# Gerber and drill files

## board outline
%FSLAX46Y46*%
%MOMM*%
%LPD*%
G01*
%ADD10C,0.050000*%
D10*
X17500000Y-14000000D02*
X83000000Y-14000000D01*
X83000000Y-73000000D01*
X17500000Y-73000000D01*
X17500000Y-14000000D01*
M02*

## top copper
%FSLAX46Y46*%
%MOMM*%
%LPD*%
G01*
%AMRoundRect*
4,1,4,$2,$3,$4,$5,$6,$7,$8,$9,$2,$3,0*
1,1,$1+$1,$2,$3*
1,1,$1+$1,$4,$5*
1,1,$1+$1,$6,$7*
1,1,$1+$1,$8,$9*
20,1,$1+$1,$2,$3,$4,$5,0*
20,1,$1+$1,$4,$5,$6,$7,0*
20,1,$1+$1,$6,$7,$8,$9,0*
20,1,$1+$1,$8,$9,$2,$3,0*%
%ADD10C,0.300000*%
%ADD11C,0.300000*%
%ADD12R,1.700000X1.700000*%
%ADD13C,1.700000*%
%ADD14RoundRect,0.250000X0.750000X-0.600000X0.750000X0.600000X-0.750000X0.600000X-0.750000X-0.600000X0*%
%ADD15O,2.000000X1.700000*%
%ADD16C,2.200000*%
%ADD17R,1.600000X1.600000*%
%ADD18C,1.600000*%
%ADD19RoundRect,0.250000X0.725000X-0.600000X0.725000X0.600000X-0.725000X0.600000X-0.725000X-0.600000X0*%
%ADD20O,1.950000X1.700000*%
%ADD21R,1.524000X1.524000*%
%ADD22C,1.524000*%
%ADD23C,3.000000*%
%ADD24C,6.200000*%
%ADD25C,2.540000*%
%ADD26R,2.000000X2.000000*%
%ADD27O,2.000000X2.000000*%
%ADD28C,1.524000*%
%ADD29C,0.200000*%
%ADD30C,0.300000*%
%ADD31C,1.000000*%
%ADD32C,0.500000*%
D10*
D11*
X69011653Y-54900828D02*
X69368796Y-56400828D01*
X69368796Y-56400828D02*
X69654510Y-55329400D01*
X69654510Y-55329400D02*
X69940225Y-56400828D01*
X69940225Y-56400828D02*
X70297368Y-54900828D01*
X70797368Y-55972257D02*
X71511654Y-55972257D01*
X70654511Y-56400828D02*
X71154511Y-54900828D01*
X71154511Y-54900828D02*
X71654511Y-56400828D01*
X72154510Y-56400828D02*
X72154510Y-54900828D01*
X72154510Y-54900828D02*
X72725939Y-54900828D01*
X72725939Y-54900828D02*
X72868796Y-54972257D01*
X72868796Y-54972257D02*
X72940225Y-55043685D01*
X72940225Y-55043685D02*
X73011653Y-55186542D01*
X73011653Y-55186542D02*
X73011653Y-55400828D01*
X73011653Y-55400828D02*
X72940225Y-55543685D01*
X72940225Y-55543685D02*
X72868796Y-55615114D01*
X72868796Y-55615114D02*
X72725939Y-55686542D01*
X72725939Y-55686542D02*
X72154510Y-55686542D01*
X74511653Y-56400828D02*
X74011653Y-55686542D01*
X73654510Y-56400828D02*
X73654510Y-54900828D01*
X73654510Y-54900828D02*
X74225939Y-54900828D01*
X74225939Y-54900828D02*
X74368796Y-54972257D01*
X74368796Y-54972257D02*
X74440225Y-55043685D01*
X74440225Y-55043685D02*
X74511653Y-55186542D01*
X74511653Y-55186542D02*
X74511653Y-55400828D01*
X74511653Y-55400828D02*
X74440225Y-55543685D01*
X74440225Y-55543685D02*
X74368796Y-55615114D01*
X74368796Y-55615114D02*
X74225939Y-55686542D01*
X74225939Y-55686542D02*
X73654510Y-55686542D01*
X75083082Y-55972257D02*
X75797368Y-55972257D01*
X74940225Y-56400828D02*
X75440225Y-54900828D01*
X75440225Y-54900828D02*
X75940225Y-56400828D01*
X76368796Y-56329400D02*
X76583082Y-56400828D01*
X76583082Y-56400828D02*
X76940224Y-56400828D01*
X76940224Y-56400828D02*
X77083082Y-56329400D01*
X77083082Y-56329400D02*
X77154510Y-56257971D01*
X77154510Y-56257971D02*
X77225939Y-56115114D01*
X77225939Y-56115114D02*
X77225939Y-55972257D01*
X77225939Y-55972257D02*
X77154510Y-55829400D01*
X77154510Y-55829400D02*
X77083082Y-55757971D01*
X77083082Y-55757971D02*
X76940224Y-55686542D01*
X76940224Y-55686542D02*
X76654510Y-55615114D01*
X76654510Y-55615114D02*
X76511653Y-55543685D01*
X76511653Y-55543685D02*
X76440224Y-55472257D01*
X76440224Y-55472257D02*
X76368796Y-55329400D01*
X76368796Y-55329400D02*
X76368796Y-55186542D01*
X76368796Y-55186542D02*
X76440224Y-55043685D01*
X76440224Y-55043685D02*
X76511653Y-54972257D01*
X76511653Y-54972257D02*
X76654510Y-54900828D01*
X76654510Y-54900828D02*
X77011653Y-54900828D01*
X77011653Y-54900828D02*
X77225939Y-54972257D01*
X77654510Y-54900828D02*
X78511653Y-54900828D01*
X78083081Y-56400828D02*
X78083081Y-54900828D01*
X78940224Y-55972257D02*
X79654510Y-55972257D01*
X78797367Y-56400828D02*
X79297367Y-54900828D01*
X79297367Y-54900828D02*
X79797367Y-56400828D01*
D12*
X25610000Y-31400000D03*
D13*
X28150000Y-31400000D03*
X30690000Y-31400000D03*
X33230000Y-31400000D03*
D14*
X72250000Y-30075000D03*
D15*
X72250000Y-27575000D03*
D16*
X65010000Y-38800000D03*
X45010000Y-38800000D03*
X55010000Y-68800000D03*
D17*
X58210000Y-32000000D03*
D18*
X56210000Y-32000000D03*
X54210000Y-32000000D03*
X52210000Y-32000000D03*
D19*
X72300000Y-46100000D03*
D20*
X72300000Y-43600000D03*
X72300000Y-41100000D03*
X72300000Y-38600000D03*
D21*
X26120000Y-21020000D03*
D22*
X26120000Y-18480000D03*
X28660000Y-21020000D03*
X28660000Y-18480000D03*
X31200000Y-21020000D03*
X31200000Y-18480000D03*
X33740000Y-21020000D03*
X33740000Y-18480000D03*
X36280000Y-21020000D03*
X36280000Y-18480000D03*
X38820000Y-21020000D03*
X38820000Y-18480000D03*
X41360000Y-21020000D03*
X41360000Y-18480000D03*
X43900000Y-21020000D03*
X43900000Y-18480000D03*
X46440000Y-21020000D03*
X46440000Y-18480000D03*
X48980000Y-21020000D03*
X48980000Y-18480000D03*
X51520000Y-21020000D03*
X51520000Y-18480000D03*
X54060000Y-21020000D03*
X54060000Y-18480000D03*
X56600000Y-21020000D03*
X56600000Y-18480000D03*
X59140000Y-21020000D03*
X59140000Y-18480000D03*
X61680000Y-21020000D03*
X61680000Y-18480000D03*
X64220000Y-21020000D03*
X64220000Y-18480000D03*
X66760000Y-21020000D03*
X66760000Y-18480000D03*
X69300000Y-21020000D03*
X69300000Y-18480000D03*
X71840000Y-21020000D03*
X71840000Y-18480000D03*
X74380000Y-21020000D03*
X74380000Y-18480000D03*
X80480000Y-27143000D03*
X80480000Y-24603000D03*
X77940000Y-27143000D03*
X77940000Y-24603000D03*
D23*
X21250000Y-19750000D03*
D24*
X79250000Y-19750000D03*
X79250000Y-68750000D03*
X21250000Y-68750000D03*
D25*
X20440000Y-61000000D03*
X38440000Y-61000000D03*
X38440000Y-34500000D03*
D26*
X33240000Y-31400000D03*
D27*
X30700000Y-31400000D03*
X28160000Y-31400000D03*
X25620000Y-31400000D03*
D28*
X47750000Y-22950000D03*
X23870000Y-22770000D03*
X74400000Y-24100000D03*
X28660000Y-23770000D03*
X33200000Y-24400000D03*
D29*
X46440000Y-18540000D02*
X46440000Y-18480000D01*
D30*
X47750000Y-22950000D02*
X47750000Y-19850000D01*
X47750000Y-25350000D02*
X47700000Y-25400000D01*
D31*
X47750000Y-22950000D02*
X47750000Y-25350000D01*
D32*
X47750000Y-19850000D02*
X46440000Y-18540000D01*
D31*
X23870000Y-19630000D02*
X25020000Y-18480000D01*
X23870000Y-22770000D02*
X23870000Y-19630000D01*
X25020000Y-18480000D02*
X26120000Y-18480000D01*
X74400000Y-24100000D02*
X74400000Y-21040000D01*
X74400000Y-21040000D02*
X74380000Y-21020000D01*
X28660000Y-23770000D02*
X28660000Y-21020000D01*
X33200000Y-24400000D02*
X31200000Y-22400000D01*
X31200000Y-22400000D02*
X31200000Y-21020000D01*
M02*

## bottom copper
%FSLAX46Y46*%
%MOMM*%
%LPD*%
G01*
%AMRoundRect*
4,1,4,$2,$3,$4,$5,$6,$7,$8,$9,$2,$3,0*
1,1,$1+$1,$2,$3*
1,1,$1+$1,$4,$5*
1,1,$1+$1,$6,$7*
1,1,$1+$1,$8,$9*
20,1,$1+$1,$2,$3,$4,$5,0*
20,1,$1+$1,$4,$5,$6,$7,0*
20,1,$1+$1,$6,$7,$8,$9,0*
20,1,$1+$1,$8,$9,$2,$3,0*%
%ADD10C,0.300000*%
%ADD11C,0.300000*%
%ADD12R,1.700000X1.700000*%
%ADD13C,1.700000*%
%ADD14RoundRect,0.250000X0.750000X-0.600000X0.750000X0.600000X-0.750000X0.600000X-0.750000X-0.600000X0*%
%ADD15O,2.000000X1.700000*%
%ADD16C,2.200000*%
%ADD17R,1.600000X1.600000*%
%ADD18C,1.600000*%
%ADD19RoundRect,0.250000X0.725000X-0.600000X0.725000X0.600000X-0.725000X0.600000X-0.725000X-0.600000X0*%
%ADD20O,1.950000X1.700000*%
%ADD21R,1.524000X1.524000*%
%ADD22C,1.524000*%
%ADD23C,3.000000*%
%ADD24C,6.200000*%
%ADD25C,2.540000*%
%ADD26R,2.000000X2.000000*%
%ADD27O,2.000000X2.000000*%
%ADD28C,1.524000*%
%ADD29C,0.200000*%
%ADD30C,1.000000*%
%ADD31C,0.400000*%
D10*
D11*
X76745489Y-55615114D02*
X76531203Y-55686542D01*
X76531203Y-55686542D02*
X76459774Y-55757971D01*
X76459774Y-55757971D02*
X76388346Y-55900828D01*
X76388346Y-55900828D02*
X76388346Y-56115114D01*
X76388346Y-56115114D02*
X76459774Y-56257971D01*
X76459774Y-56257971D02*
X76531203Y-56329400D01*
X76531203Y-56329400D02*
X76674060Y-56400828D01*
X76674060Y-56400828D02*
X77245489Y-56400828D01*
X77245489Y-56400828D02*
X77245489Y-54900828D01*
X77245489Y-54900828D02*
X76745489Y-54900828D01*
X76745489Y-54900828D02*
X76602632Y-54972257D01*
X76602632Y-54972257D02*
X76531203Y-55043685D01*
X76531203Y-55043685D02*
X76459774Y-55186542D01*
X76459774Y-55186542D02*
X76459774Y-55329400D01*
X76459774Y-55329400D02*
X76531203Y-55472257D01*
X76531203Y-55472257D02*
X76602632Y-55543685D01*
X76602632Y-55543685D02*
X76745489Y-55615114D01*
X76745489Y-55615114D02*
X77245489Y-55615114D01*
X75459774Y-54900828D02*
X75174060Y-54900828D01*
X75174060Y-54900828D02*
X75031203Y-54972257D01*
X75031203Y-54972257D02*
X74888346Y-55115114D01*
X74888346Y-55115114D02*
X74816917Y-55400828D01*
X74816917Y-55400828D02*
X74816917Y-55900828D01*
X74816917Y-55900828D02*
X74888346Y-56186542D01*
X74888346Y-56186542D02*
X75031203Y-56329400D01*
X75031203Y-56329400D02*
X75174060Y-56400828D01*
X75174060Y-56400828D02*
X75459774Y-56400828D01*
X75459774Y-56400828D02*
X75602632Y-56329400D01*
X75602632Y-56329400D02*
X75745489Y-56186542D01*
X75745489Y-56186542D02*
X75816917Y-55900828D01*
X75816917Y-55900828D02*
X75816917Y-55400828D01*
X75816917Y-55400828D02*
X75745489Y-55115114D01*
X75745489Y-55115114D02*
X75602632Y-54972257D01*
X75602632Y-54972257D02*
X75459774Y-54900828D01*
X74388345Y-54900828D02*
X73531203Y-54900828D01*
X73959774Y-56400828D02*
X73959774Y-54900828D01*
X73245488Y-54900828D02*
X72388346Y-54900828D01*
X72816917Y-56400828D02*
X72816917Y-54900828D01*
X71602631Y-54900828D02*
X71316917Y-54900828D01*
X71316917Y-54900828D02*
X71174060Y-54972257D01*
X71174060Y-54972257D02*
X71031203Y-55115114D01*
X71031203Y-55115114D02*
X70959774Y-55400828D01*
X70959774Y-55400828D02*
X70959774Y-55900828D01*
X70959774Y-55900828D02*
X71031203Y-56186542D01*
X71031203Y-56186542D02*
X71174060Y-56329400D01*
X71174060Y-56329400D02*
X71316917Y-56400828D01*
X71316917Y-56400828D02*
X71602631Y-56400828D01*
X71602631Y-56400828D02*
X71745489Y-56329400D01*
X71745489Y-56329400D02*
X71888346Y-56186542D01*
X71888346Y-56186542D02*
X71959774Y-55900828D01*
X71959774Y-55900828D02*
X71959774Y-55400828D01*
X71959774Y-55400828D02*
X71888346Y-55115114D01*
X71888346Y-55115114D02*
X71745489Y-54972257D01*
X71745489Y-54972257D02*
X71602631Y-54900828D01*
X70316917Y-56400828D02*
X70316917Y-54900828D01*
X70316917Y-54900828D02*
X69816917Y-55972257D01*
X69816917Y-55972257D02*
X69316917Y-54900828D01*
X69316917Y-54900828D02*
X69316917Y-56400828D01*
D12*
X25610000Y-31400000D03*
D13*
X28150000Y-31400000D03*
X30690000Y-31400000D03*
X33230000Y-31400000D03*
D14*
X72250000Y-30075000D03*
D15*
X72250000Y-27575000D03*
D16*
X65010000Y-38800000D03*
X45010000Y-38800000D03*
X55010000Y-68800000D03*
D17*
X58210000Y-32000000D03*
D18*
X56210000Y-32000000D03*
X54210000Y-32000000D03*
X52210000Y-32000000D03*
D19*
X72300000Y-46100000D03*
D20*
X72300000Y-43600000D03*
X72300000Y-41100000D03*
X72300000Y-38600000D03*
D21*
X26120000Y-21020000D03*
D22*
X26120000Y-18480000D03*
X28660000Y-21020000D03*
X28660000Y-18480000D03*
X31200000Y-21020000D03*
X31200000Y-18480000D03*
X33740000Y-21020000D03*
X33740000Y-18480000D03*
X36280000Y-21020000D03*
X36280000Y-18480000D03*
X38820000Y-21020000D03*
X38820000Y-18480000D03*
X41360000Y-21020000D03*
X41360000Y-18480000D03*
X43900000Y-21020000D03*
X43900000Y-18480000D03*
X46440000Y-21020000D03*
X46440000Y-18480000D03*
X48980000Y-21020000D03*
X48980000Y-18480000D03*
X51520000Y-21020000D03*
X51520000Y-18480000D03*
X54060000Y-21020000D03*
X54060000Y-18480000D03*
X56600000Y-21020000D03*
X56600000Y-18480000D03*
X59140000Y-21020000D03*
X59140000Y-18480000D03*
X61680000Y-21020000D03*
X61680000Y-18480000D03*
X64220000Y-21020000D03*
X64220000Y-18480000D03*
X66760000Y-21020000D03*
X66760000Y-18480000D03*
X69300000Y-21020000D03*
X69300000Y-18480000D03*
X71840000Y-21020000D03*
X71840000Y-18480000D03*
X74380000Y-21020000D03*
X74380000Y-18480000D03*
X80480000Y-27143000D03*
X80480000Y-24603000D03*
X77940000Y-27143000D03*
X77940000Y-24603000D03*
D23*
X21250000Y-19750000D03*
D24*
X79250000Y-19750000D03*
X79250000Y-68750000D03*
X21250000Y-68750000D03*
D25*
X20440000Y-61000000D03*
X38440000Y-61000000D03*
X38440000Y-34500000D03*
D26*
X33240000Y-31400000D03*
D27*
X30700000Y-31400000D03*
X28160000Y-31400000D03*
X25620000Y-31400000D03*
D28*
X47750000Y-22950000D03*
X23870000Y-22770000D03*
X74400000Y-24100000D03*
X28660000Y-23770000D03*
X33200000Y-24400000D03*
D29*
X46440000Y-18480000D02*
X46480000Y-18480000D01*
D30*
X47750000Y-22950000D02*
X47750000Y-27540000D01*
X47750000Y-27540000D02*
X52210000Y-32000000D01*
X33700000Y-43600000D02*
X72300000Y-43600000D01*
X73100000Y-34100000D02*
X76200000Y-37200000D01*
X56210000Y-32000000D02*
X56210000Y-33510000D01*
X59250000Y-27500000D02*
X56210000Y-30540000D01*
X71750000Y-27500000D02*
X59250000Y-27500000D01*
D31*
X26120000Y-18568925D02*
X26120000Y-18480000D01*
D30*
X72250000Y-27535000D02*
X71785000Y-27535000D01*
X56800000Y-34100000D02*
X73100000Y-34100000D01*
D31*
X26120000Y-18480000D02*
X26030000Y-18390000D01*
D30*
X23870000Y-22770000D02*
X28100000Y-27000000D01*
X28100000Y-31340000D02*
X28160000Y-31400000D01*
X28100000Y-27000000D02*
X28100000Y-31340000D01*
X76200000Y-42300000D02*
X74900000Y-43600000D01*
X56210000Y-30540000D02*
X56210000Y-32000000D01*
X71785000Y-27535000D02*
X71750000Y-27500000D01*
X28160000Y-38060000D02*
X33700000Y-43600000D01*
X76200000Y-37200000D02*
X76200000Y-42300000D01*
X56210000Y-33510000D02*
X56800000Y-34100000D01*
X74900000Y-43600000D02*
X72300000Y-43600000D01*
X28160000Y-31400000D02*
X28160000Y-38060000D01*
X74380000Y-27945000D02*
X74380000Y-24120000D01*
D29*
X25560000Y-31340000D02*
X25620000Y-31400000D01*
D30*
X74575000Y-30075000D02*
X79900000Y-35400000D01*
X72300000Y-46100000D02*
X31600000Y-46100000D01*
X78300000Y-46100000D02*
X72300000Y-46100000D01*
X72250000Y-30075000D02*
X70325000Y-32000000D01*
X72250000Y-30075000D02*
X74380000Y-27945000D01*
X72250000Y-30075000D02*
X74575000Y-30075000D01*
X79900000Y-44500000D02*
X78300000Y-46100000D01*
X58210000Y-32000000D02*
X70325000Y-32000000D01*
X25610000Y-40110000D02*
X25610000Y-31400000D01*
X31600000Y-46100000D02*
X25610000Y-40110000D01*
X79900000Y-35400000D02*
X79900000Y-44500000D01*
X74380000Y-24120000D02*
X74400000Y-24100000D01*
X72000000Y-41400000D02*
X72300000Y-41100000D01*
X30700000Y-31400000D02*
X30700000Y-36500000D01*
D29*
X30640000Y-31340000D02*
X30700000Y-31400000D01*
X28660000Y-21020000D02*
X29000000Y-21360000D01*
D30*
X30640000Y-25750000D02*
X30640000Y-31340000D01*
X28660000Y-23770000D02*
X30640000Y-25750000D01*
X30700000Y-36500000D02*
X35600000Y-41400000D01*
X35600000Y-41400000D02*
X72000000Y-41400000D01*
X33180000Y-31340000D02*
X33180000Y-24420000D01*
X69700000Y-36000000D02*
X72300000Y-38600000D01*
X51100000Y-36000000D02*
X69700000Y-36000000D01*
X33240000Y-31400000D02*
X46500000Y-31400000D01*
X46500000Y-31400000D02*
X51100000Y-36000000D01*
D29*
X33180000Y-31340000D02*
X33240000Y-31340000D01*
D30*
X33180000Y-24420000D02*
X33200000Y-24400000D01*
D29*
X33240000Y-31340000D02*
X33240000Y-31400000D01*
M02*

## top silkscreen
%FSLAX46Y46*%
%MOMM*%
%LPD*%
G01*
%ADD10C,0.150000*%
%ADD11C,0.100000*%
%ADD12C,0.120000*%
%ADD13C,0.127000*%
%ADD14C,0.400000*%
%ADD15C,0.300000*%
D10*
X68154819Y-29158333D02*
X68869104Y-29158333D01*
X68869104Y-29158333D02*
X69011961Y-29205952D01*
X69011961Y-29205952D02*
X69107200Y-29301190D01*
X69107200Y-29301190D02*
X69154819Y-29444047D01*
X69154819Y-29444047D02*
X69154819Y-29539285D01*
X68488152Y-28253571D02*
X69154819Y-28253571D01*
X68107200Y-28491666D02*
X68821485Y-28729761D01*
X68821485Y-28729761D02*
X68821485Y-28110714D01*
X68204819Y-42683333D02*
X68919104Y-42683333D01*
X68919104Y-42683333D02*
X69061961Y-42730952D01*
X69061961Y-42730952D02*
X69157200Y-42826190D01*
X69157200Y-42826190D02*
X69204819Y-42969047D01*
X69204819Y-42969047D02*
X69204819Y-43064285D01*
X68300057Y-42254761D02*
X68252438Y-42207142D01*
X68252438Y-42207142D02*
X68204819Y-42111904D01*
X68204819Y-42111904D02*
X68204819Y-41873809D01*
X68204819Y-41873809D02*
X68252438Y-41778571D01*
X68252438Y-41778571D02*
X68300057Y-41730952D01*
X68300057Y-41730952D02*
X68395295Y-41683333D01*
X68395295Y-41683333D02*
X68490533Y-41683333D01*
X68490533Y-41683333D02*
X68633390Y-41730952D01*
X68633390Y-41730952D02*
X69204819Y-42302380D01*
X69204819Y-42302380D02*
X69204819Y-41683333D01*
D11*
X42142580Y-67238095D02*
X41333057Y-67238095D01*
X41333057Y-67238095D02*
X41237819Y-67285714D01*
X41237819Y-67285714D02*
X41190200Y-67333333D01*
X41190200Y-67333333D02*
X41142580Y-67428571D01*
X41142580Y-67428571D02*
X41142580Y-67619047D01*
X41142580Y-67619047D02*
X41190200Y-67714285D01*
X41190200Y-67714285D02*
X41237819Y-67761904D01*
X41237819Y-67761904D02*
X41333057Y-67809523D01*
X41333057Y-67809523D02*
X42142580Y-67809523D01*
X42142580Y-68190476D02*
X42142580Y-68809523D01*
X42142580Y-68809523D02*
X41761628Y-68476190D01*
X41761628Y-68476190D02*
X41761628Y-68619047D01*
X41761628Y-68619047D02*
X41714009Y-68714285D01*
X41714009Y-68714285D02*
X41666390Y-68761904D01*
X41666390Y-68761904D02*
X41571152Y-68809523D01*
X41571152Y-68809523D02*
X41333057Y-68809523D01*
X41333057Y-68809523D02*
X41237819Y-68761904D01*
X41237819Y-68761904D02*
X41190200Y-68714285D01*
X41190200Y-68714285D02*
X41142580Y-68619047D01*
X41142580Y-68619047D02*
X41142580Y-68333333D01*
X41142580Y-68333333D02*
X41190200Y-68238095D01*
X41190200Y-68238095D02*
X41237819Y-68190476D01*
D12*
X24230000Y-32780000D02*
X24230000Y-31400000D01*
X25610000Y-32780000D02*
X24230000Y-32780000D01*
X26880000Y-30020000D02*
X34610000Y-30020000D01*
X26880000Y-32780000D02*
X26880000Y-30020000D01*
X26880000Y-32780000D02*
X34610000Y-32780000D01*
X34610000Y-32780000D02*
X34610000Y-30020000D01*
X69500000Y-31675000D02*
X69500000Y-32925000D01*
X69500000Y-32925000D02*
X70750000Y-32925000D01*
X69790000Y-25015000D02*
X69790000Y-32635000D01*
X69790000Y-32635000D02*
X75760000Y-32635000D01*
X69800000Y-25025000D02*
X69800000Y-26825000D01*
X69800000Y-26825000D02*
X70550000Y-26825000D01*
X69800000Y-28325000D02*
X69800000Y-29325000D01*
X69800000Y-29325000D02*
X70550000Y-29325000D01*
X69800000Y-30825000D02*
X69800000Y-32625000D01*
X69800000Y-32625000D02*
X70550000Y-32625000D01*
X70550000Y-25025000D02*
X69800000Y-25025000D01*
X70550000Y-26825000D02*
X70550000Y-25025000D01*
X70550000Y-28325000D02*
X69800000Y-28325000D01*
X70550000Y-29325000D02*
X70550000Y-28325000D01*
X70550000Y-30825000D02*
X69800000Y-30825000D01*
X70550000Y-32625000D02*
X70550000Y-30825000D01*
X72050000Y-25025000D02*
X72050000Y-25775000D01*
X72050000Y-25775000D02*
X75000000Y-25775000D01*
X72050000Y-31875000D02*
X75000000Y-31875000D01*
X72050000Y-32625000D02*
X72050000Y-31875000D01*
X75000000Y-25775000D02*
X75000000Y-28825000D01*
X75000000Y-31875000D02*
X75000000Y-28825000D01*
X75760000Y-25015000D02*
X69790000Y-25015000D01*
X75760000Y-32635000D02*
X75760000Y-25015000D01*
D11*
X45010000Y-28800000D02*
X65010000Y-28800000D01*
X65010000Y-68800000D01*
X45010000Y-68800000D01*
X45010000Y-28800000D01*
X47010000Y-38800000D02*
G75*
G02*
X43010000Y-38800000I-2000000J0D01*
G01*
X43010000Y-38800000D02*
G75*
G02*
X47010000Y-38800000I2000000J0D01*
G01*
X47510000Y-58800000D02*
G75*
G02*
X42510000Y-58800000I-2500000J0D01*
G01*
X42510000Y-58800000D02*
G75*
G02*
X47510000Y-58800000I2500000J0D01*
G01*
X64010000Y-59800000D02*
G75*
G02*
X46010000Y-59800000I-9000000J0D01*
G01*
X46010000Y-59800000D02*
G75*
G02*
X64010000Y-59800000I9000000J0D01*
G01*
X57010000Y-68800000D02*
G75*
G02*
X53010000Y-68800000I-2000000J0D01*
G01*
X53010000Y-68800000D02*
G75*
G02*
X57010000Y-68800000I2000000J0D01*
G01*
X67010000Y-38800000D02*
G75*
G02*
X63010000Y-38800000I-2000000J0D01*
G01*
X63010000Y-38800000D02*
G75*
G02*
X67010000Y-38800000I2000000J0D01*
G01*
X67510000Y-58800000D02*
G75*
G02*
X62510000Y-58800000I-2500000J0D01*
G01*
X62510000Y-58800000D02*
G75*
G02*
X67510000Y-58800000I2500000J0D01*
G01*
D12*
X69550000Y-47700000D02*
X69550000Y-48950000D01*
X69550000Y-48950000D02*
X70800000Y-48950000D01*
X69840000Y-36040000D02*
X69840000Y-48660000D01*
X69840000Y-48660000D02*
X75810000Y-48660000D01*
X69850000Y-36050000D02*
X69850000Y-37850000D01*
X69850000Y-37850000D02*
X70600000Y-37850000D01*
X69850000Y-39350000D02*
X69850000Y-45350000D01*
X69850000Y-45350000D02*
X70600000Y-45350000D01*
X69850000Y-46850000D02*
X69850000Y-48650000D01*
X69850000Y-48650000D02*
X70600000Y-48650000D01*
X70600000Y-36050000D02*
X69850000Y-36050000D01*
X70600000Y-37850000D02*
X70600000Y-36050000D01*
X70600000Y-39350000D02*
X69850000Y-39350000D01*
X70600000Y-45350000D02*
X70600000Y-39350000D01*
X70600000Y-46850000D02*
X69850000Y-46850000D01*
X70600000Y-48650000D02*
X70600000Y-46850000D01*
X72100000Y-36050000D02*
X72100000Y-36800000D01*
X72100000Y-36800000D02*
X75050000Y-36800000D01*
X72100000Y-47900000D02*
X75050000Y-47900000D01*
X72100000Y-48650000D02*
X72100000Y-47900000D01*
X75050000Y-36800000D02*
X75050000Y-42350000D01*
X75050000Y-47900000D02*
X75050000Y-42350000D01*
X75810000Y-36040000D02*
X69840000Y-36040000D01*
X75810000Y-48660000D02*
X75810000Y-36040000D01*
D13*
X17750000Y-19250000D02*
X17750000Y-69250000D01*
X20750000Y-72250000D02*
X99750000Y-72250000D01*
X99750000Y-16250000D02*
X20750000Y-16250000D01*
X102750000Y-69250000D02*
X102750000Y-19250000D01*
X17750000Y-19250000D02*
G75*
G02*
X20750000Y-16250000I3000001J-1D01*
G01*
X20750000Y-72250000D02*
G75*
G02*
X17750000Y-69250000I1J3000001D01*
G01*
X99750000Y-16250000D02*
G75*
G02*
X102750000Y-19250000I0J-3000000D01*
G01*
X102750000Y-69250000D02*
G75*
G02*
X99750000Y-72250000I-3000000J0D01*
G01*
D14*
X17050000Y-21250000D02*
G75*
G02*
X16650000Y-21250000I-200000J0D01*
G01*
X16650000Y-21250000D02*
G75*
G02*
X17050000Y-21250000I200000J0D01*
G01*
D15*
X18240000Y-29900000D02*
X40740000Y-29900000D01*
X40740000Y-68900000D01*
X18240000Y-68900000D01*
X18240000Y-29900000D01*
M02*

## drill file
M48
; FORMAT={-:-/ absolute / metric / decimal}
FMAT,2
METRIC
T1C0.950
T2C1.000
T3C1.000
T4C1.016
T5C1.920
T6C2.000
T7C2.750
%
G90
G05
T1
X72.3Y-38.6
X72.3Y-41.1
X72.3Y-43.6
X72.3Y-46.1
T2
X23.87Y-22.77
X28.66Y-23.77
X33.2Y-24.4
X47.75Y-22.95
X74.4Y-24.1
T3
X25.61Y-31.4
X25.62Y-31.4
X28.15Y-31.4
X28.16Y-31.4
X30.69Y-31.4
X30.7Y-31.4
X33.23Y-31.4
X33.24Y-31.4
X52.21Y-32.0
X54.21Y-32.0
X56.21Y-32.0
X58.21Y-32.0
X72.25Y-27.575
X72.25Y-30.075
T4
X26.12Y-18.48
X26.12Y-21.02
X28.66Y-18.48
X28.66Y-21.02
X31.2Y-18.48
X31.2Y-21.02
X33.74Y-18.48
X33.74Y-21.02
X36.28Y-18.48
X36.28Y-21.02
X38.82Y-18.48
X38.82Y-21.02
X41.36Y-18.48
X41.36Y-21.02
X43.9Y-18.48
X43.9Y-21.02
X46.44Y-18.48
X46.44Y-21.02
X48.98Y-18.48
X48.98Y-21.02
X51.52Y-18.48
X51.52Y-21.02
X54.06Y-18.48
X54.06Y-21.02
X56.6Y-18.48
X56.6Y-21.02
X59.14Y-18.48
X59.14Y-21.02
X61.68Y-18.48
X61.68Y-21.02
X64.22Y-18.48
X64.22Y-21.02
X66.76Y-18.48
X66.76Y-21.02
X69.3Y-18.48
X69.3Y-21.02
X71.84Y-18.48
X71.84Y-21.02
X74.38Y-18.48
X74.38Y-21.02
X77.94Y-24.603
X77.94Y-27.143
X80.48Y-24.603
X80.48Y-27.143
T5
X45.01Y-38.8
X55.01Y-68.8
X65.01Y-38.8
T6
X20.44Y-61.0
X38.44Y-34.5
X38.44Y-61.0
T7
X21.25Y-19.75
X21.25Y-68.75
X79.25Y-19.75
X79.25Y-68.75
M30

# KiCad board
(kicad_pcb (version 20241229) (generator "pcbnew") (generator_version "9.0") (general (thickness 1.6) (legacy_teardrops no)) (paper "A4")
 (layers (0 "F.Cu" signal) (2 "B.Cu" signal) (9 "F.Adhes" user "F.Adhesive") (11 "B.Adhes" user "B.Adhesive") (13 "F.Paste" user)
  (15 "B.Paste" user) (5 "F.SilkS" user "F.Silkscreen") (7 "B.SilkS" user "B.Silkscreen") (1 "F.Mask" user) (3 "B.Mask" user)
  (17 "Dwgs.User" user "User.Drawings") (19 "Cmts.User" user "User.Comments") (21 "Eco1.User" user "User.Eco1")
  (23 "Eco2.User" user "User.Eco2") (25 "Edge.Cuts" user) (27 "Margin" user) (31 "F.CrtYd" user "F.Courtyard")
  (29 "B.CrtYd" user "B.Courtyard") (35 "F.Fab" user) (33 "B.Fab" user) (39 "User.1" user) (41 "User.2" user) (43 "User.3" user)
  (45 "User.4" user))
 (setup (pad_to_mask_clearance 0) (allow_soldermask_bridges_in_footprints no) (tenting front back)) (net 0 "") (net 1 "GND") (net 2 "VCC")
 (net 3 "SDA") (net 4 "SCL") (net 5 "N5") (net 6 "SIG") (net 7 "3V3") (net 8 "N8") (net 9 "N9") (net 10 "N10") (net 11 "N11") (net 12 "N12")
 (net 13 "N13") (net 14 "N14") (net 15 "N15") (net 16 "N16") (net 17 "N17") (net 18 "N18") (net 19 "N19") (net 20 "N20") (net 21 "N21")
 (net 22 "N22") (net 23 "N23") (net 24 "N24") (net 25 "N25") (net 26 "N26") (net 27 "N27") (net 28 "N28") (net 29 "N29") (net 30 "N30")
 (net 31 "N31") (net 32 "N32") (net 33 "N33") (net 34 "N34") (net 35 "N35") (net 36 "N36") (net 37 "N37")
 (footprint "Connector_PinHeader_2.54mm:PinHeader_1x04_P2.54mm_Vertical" (layer "F.Cu") (at 25.61 31.4 90)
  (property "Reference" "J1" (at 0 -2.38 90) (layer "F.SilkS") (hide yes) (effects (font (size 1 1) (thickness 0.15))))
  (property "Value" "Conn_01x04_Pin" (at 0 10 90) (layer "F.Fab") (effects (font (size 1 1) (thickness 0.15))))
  (fp_line (start -1.38 -1.38) (end 0 -1.38) (stroke (width 0.12) (type solid)) (layer "F.SilkS"))
  (fp_line (start -1.38 0) (end -1.38 -1.38) (stroke (width 0.12) (type solid)) (layer "F.SilkS"))
  (fp_line (start 1.38 1.27) (end 1.38 9) (stroke (width 0.12) (type solid)) (layer "F.SilkS"))
  (fp_line (start -1.38 1.27) (end 1.38 1.27) (stroke (width 0.12) (type solid)) (layer "F.SilkS"))
  (fp_line (start -1.38 1.27) (end -1.38 9) (stroke (width 0.12) (type solid)) (layer "F.SilkS"))
  (fp_line (start -1.38 9) (end 1.38 9) (stroke (width 0.12) (type solid)) (layer "F.SilkS"))
  (pad "1" thru_hole rect (at 0 0 90) (size 1.7 1.7) (drill 1) (layers "*.Cu" "*.Mask") (remove_unused_layers no) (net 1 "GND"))
  (pad "2" thru_hole circle (at 0 2.54 90) (size 1.7 1.7) (drill 1) (layers "*.Cu" "*.Mask") (remove_unused_layers no) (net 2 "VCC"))
  (pad "3" thru_hole circle (at 0 5.08 90) (size 1.7 1.7) (drill 1) (layers "*.Cu" "*.Mask") (remove_unused_layers no) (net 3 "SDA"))
  (pad "4" thru_hole circle (at 0 7.62 90) (size 1.7 1.7) (drill 1) (layers "*.Cu" "*.Mask") (remove_unused_layers no) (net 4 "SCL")))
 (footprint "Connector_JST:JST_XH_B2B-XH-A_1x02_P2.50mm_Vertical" (layer "F.Cu") (at 72.25 30.075 90)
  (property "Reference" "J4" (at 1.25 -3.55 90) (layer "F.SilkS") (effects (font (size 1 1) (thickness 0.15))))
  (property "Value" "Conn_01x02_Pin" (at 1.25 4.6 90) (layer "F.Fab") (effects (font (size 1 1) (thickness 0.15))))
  (fp_line (start -1.6 -2.75) (end -2.85 -2.75) (stroke (width 0.12) (type solid)) (layer "F.SilkS"))
  (fp_line (start -2.85 -2.75) (end -2.85 -1.5) (stroke (width 0.12) (type solid)) (layer "F.SilkS"))
  (fp_line (start 5.06 -2.46) (end -2.56 -2.46) (stroke (width 0.12) (type solid)) (layer "F.SilkS"))
  (fp_line (start -2.56 -2.46) (end -2.56 3.51) (stroke (width 0.12) (type solid)) (layer "F.SilkS"))
  (fp_line (start 5.05 -2.45) (end 3.25 -2.45) (stroke (width 0.12) (type solid)) (layer "F.SilkS"))
  (fp_line (start 3.25 -2.45) (end 3.25 -1.7) (stroke (width 0.12) (type solid)) (layer "F.SilkS"))
  (fp_line (start 1.75 -2.45) (end 0.75 -2.45) (stroke (width 0.12) (type solid)) (layer "F.SilkS"))
  (fp_line (start 0.75 -2.45) (end 0.75 -1.7) (stroke (width 0.12) (type solid)) (layer "F.SilkS"))
  (fp_line (start -0.75 -2.45) (end -2.55 -2.45) (stroke (width 0.12) (type solid)) (layer "F.SilkS"))
  (fp_line (start -2.55 -2.45) (end -2.55 -1.7) (stroke (width 0.12) (type solid)) (layer "F.SilkS"))
  (fp_line (start 5.05 -1.7) (end 5.05 -2.45) (stroke (width 0.12) (type solid)) (layer "F.SilkS"))
  (fp_line (start 3.25 -1.7) (end 5.05 -1.7) (stroke (width 0.12) (type solid)) (layer "F.SilkS"))
  (fp_line (start 1.75 -1.7) (end 1.75 -2.45) (stroke (width 0.12) (type solid)) (layer "F.SilkS"))
  (fp_line (start 0.75 -1.7) (end 1.75 -1.7) (stroke (width 0.12) (type solid)) (layer "F.SilkS"))
  (fp_line (start -0.75 -1.7) (end -0.75 -2.45) (stroke (width 0.12) (type solid)) (layer "F.SilkS"))
  (fp_line (start -2.55 -1.7) (end -0.75 -1.7) (stroke (width 0.12) (type solid)) (layer "F.SilkS"))
  (fp_line (start 5.05 -0.2) (end 4.3 -0.2) (stroke (width 0.12) (type solid)) (layer "F.SilkS"))
  (fp_line (start 4.3 -0.2) (end 4.3 2.75) (stroke (width 0.12) (type solid)) (layer "F.SilkS"))
  (fp_line (start -1.8 -0.2) (end -1.8 2.75) (stroke (width 0.12) (type solid)) (layer "F.SilkS"))
  (fp_line (start -2.55 -0.2) (end -1.8 -0.2) (stroke (width 0.12) (type solid)) (layer "F.SilkS"))
  (fp_line (start 4.3 2.75) (end 1.25 2.75) (stroke (width 0.12) (type solid)) (layer "F.SilkS"))
  (fp_line (start -1.8 2.75) (end 1.25 2.75) (stroke (width 0.12) (type solid)) (layer "F.SilkS"))
  (fp_line (start 5.06 3.51) (end 5.06 -2.46) (stroke (width 0.12) (type solid)) (layer "F.SilkS"))
  (fp_line (start -2.56 3.51) (end 5.06 3.51) (stroke (width 0.12) (type solid)) (layer "F.SilkS"))
  (pad "1" thru_hole roundrect (at 0 0 90) (size 1.7 2) (drill 1) (layers "*.Cu" "*.Mask") (remove_unused_layers no)
   (roundrect_rratio 0.147059) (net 1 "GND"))
  (pad "2" thru_hole oval (at 2.5 0 90) (size 1.7 2) (drill 1) (layers "*.Cu" "*.Mask") (remove_unused_layers no) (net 2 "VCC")))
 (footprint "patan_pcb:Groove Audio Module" (layer "F.Cu") (at 65.01 28.8 -90)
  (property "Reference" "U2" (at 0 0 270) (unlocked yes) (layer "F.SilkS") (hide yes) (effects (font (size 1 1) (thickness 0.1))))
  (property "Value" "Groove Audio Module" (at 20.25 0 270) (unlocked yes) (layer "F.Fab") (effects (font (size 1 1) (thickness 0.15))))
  (fp_rect (start 0 0) (end 40 20) (stroke (width 0.1) (type solid)) (fill no) (layer "F.SilkS"))
  (fp_circle (center 10 20) (end 12 20) (stroke (width 0.1) (type default)) (fill no) (layer "F.SilkS"))
  (fp_circle (center 30 20) (end 32.5 20) (stroke (width 0.1) (type solid)) (fill no) (layer "F.SilkS"))
  (fp_circle (center 31 10) (end 40 10) (stroke (width 0.1) (type solid)) (fill no) (layer "F.SilkS"))
  (fp_circle (center 40 10) (end 42 10) (stroke (width 0.1) (type default)) (fill no) (layer "F.SilkS"))
  (fp_circle (center 10 0) (end 12 0) (stroke (width 0.1) (type default)) (fill no) (layer "F.SilkS"))
  (fp_circle (center 30 0) (end 32.5 0) (stroke (width 0.1) (type solid)) (fill no) (layer "F.SilkS"))
  (pad "" thru_hole circle (at 10 0 270) (size 2.2 2.2) (drill 1.92) (layers "*.Cu" "*.Mask") (remove_unused_layers no)
   (solder_mask_margin 0.127))
  (pad "" thru_hole circle (at 10 20 270) (size 2.2 2.2) (drill 1.92) (layers "*.Cu" "*.Mask") (remove_unused_layers no)
   (solder_mask_margin 0.127))
  (pad "" thru_hole circle (at 40 10 270) (size 2.2 2.2) (drill 1.92) (layers "*.Cu" "*.Mask") (remove_unused_layers no)
   (solder_mask_margin 0.127))
  (pad "1" thru_hole rect (at 3.2 6.8 270) (size 1.6 1.6) (drill 1) (layers "*.Cu" "*.Mask") (remove_unused_layers no) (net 1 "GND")
   (solder_mask_margin 0.127))
  (pad "2" thru_hole circle (at 3.2 8.8 270) (size 1.6 1.6) (drill 1) (layers "*.Cu" "*.Mask") (remove_unused_layers no) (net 2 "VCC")
   (solder_mask_margin 0.127))
  (pad "3" thru_hole circle (at 3.2 10.8 270) (size 1.6 1.6) (drill 1) (layers "*.Cu" "*.Mask") (remove_unused_layers no) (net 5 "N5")
   (solder_mask_margin 0.127))
  (pad "4" thru_hole circle (at 3.2 12.8 270) (size 1.6 1.6) (drill 1) (layers "*.Cu" "*.Mask") (remove_unused_layers no) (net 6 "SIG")
   (solder_mask_margin 0.127)))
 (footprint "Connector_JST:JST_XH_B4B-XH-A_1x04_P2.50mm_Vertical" (layer "F.Cu") (at 72.3 46.1 90)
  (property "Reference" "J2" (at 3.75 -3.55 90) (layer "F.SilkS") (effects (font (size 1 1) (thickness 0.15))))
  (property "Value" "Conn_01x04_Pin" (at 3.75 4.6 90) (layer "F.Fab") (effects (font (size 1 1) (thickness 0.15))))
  (fp_line (start -1.6 -2.75) (end -2.85 -2.75) (stroke (width 0.12) (type solid)) (layer "F.SilkS"))
  (fp_line (start -2.85 -2.75) (end -2.85 -1.5) (stroke (width 0.12) (type solid)) (layer "F.SilkS"))
  (fp_line (start 10.06 -2.46) (end -2.56 -2.46) (stroke (width 0.12) (type solid)) (layer "F.SilkS"))
  (fp_line (start -2.56 -2.46) (end -2.56 3.51) (stroke (width 0.12) (type solid)) (layer "F.SilkS"))
  (fp_line (start 10.05 -2.45) (end 8.25 -2.45) (stroke (width 0.12) (type solid)) (layer "F.SilkS"))
  (fp_line (start 8.25 -2.45) (end 8.25 -1.7) (stroke (width 0.12) (type solid)) (layer "F.SilkS"))
  (fp_line (start 6.75 -2.45) (end 0.75 -2.45) (stroke (width 0.12) (type solid)) (layer "F.SilkS"))
  (fp_line (start 0.75 -2.45) (end 0.75 -1.7) (stroke (width 0.12) (type solid)) (layer "F.SilkS"))
  (fp_line (start -0.75 -2.45) (end -2.55 -2.45) (stroke (width 0.12) (type solid)) (layer "F.SilkS"))
  (fp_line (start -2.55 -2.45) (end -2.55 -1.7) (stroke (width 0.12) (type solid)) (layer "F.SilkS"))
  (fp_line (start 10.05 -1.7) (end 10.05 -2.45) (stroke (width 0.12) (type solid)) (layer "F.SilkS"))
  (fp_line (start 8.25 -1.7) (end 10.05 -1.7) (stroke (width 0.12) (type solid)) (layer "F.SilkS"))
  (fp_line (start 6.75 -1.7) (end 6.75 -2.45) (stroke (width 0.12) (type solid)) (layer "F.SilkS"))
  (fp_line (start 0.75 -1.7) (end 6.75 -1.7) (stroke (width 0.12) (type solid)) (layer "F.SilkS"))
  (fp_line (start -0.75 -1.7) (end -0.75 -2.45) (stroke (width 0.12) (type solid)) (layer "F.SilkS"))
  (fp_line (start -2.55 -1.7) (end -0.75 -1.7) (stroke (width 0.12) (type solid)) (layer "F.SilkS"))
  (fp_line (start 10.05 -0.2) (end 9.3 -0.2) (stroke (width 0.12) (type solid)) (layer "F.SilkS"))
  (fp_line (start 9.3 -0.2) (end 9.3 2.75) (stroke (width 0.12) (type solid)) (layer "F.SilkS"))
  (fp_line (start -1.8 -0.2) (end -1.8 2.75) (stroke (width 0.12) (type solid)) (layer "F.SilkS"))
  (fp_line (start -2.55 -0.2) (end -1.8 -0.2) (stroke (width 0.12) (type solid)) (layer "F.SilkS"))
  (fp_line (start 9.3 2.75) (end 3.75 2.75) (stroke (width 0.12) (type solid)) (layer "F.SilkS"))
  (fp_line (start -1.8 2.75) (end 3.75 2.75) (stroke (width 0.12) (type solid)) (layer "F.SilkS"))
  (fp_line (start 10.06 3.51) (end 10.06 -2.46) (stroke (width 0.12) (type solid)) (layer "F.SilkS"))
  (fp_line (start -2.56 3.51) (end 10.06 3.51) (stroke (width 0.12) (type solid)) (layer "F.SilkS"))
  (pad "1" thru_hole roundrect (at 0 0 90) (size 1.7 1.95) (drill 0.95) (layers "*.Cu" "*.Mask") (remove_unused_layers no)
   (roundrect_rratio 0.147059) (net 1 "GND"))
  (pad "2" thru_hole oval (at 2.5 0 90) (size 1.7 1.95) (drill 0.95) (layers "*.Cu" "*.Mask") (remove_unused_layers no) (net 2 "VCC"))
  (pad "3" thru_hole oval (at 5 0 90) (size 1.7 1.95) (drill 0.95) (layers "*.Cu" "*.Mask") (remove_unused_layers no) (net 3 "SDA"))
  (pad "4" thru_hole oval (at 7.5 0 90) (size 1.7 1.95) (drill 0.95) (layers "*.Cu" "*.Mask") (remove_unused_layers no) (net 4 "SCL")))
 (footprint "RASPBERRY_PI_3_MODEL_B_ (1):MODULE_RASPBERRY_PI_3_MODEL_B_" (layer "F.Cu") (at 60.25 44.25)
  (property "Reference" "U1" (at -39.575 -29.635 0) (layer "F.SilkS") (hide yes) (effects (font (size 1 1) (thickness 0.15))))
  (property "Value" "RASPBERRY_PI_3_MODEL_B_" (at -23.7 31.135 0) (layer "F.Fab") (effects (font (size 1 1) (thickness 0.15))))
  (fp_line (start -42.5 -25) (end -42.5 25) (stroke (width 0.127) (type solid)) (layer "F.SilkS"))
  (fp_line (start -39.5 28) (end 39.5 28) (stroke (width 0.127) (type solid)) (layer "F.SilkS"))
  (fp_line (start 39.5 -28) (end -39.5 -28) (stroke (width 0.127) (type solid)) (layer "F.SilkS"))
  (fp_line (start 42.5 25) (end 42.5 -25) (stroke (width 0.127) (type solid)) (layer "F.SilkS"))
  (fp_arc (start -42.5 -25) (mid -41.62132 -27.12132) (end -39.5 -28) (stroke (width 0.127) (type solid)) (layer "F.SilkS"))
  (fp_arc (start -39.5 28) (mid -41.62132 27.12132) (end -42.5 25) (stroke (width 0.127) (type solid)) (layer "F.SilkS"))
  (fp_arc (start 39.5 -28) (mid 41.62132 -27.12132) (end 42.5 -25) (stroke (width 0.127) (type solid)) (layer "F.SilkS"))
  (fp_arc (start 42.5 25) (mid 41.62132 27.12132) (end 39.5 28) (stroke (width 0.127) (type solid)) (layer "F.SilkS"))
  (fp_circle (center -43.4 -23) (end -43.2 -23) (stroke (width 0.4) (type solid)) (fill no) (layer "F.SilkS"))
  (pad "1" thru_hole rect (at -34.13 -23.23) (size 1.524 1.524) (drill 1.016) (layers "*.Cu" "*.Mask") (remove_unused_layers no)
   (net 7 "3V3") (solder_mask_margin 0.102))
  (pad "2" thru_hole circle (at -34.13 -25.77) (size 1.524 1.524) (drill 1.016) (layers "*.Cu" "*.Mask") (remove_unused_layers no)
   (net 2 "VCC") (solder_mask_margin 0.102))
  (pad "3" thru_hole circle (at -31.59 -23.23) (size 1.524 1.524) (drill 1.016) (layers "*.Cu" "*.Mask") (remove_unused_layers no)
   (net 3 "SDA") (solder_mask_margin 0.102))
  (pad "4" thru_hole circle (at -31.59 -25.77) (size 1.524 1.524) (drill 1.016) (layers "*.Cu" "*.Mask") (remove_unused_layers no)
   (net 2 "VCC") (solder_mask_margin 0.102))
  (pad "5" thru_hole circle (at -29.05 -23.23) (size 1.524 1.524) (drill 1.016) (layers "*.Cu" "*.Mask") (remove_unused_layers no)
   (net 4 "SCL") (solder_mask_margin 0.102))
  (pad "6" thru_hole circle (at -29.05 -25.77) (size 1.524 1.524) (drill 1.016) (layers "*.Cu" "*.Mask") (remove_unused_layers no)
   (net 1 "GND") (solder_mask_margin 0.102))
  (pad "7" thru_hole circle (at -26.51 -23.23) (size 1.524 1.524) (drill 1.016) (layers "*.Cu" "*.Mask") (remove_unused_layers no)
   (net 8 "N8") (solder_mask_margin 0.102))
  (pad "8" thru_hole circle (at -26.51 -25.77) (size 1.524 1.524) (drill 1.016) (layers "*.Cu" "*.Mask") (remove_unused_layers no)
   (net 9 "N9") (solder_mask_margin 0.102))
  (pad "9" thru_hole circle (at -23.97 -23.23) (size 1.524 1.524) (drill 1.016) (layers "*.Cu" "*.Mask") (remove_unused_layers no)
   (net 1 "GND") (solder_mask_margin 0.102))
  (pad "10" thru_hole circle (at -23.97 -25.77) (size 1.524 1.524) (drill 1.016) (layers "*.Cu" "*.Mask") (remove_unused_layers no)
   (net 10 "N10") (solder_mask_margin 0.102))
  (pad "11" thru_hole circle (at -21.43 -23.23) (size 1.524 1.524) (drill 1.016) (layers "*.Cu" "*.Mask") (remove_unused_layers no)
   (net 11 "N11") (solder_mask_margin 0.102))
  (pad "12" thru_hole circle (at -21.43 -25.77) (size 1.524 1.524) (drill 1.016) (layers "*.Cu" "*.Mask") (remove_unused_layers no)
   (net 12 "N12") (solder_mask_margin 0.102))
  (pad "13" thru_hole circle (at -18.89 -23.23) (size 1.524 1.524) (drill 1.016) (layers "*.Cu" "*.Mask") (remove_unused_layers no)
   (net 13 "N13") (solder_mask_margin 0.102))
  (pad "14" thru_hole circle (at -18.89 -25.77) (size 1.524 1.524) (drill 1.016) (layers "*.Cu" "*.Mask") (remove_unused_layers no)
   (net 1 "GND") (solder_mask_margin 0.102))
  (pad "15" thru_hole circle (at -16.35 -23.23) (size 1.524 1.524) (drill 1.016) (layers "*.Cu" "*.Mask") (remove_unused_layers no)
   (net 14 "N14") (solder_mask_margin 0.102))
  (pad "16" thru_hole circle (at -16.35 -25.77) (size 1.524 1.524) (drill 1.016) (layers "*.Cu" "*.Mask") (remove_unused_layers no)
   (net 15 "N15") (solder_mask_margin 0.102))
  (pad "17" thru_hole circle (at -13.81 -23.23) (size 1.524 1.524) (drill 1.016) (layers "*.Cu" "*.Mask") (remove_unused_layers no)
   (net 7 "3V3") (solder_mask_margin 0.102))
  (pad "18" thru_hole circle (at -13.81 -25.77) (size 1.524 1.524) (drill 1.016) (layers "*.Cu" "*.Mask") (remove_unused_layers no)
   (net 6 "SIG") (solder_mask_margin 0.102))
  (pad "19" thru_hole circle (at -11.27 -23.23) (size 1.524 1.524) (drill 1.016) (layers "*.Cu" "*.Mask") (remove_unused_layers no)
   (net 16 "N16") (solder_mask_margin 0.102))
  (pad "20" thru_hole circle (at -11.27 -25.77) (size 1.524 1.524) (drill 1.016) (layers "*.Cu" "*.Mask") (remove_unused_layers no)
   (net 1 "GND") (solder_mask_margin 0.102))
  (pad "21" thru_hole circle (at -8.73 -23.23) (size 1.524 1.524) (drill 1.016) (layers "*.Cu" "*.Mask") (remove_unused_layers no)
   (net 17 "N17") (solder_mask_margin 0.102))
  (pad "22" thru_hole circle (at -8.73 -25.77) (size 1.524 1.524) (drill 1.016) (layers "*.Cu" "*.Mask") (remove_unused_layers no)
   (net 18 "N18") (solder_mask_margin 0.102))
  (pad "23" thru_hole circle (at -6.19 -23.23) (size 1.524 1.524) (drill 1.016) (layers "*.Cu" "*.Mask") (remove_unused_layers no)
   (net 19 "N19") (solder_mask_margin 0.102))
  (pad "24" thru_hole circle (at -6.19 -25.77) (size 1.524 1.524) (drill 1.016) (layers "*.Cu" "*.Mask") (remove_unused_layers no)
   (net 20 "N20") (solder_mask_margin 0.102))
  (pad "25" thru_hole circle (at -3.65 -23.23) (size 1.524 1.524) (drill 1.016) (layers "*.Cu" "*.Mask") (remove_unused_layers no)
   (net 1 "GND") (solder_mask_margin 0.102))
  (pad "26" thru_hole circle (at -3.65 -25.77) (size 1.524 1.524) (drill 1.016) (layers "*.Cu" "*.Mask") (remove_unused_layers no)
   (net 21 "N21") (solder_mask_margin 0.102))
  (pad "27" thru_hole circle (at -1.11 -23.23) (size 1.524 1.524) (drill 1.016) (layers "*.Cu" "*.Mask") (remove_unused_layers no)
   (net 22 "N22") (solder_mask_margin 0.102))
  (pad "28" thru_hole circle (at -1.11 -25.77) (size 1.524 1.524) (drill 1.016) (layers "*.Cu" "*.Mask") (remove_unused_layers no)
   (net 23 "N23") (solder_mask_margin 0.102))
  (pad "29" thru_hole circle (at 1.43 -23.23) (size 1.524 1.524) (drill 1.016) (layers "*.Cu" "*.Mask") (remove_unused_layers no)
   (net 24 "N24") (solder_mask_margin 0.102))
  (pad "30" thru_hole circle (at 1.43 -25.77) (size 1.524 1.524) (drill 1.016) (layers "*.Cu" "*.Mask") (remove_unused_layers no)
   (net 1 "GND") (solder_mask_margin 0.102))
  (pad "31" thru_hole circle (at 3.97 -23.23) (size 1.524 1.524) (drill 1.016) (layers "*.Cu" "*.Mask") (remove_unused_layers no)
   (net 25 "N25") (solder_mask_margin 0.102))
  (pad "32" thru_hole circle (at 3.97 -25.77) (size 1.524 1.524) (drill 1.016) (layers "*.Cu" "*.Mask") (remove_unused_layers no)
   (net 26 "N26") (solder_mask_margin 0.102))
  (pad "33" thru_hole circle (at 6.51 -23.23) (size 1.524 1.524) (drill 1.016) (layers "*.Cu" "*.Mask") (remove_unused_layers no)
   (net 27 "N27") (solder_mask_margin 0.102))
  (pad "34" thru_hole circle (at 6.51 -25.77) (size 1.524 1.524) (drill 1.016) (layers "*.Cu" "*.Mask") (remove_unused_layers no)
   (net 1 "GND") (solder_mask_margin 0.102))
  (pad "35" thru_hole circle (at 9.05 -23.23) (size 1.524 1.524) (drill 1.016) (layers "*.Cu" "*.Mask") (remove_unused_layers no)
   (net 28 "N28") (solder_mask_margin 0.102))
  (pad "36" thru_hole circle (at 9.05 -25.77) (size 1.524 1.524) (drill 1.016) (layers "*.Cu" "*.Mask") (remove_unused_layers no)
   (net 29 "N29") (solder_mask_margin 0.102))
  (pad "37" thru_hole circle (at 11.59 -23.23) (size 1.524 1.524) (drill 1.016) (layers "*.Cu" "*.Mask") (remove_unused_layers no)
   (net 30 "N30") (solder_mask_margin 0.102))
  (pad "38" thru_hole circle (at 11.59 -25.77) (size 1.524 1.524) (drill 1.016) (layers "*.Cu" "*.Mask") (remove_unused_layers no)
   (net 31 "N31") (solder_mask_margin 0.102))
  (pad "39" thru_hole circle (at 14.13 -23.23) (size 1.524 1.524) (drill 1.016) (layers "*.Cu" "*.Mask") (remove_unused_layers no)
   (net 1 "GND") (solder_mask_margin 0.102))
  (pad "40" thru_hole circle (at 14.13 -25.77) (size 1.524 1.524) (drill 1.016) (layers "*.Cu" "*.Mask") (remove_unused_layers no)
   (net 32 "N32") (solder_mask_margin 0.102))
  (pad "41" thru_hole circle (at 20.23 -17.107) (size 1.524 1.524) (drill 1.016) (layers "*.Cu" "*.Mask") (remove_unused_layers no)
   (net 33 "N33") (solder_mask_margin 0.102))
  (pad "42" thru_hole circle (at 20.23 -19.647) (size 1.524 1.524) (drill 1.016) (layers "*.Cu" "*.Mask") (remove_unused_layers no)
   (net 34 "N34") (solder_mask_margin 0.102))
  (pad "43" thru_hole circle (at 17.69 -17.107) (size 1.524 1.524) (drill 1.016) (layers "*.Cu" "*.Mask") (remove_unused_layers no)
   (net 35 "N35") (solder_mask_margin 0.102))
  (pad "44" thru_hole circle (at 17.69 -19.647) (size 1.524 1.524) (drill 1.016) (layers "*.Cu" "*.Mask") (remove_unused_layers no)
   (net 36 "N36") (solder_mask_margin 0.102))
  (pad "S1" thru_hole circle (at -39 -24.5) (size 3 3) (drill 2.75) (layers "*.Cu" "*.Mask") (remove_unused_layers no) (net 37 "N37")
   (solder_mask_margin 0.102))
  (pad "S2" thru_hole circle (at 19 -24.5) (size 6.2 6.2) (drill 2.75) (layers "*.Cu" "*.Mask") (remove_unused_layers no) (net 37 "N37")
   (solder_mask_margin 0.102))
  (pad "S3" thru_hole circle (at 19 24.5) (size 6.2 6.2) (drill 2.75) (layers "*.Cu" "*.Mask") (remove_unused_layers no) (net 37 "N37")
   (solder_mask_margin 0.102))
  (pad "S4" thru_hole circle (at -39 24.5) (size 6.2 6.2) (drill 2.75) (layers "*.Cu" "*.Mask") (remove_unused_layers no) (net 37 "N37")
   (solder_mask_margin 0.102)))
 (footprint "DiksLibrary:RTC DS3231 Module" (layer "B.Cu") (at 40.74 68.9 90)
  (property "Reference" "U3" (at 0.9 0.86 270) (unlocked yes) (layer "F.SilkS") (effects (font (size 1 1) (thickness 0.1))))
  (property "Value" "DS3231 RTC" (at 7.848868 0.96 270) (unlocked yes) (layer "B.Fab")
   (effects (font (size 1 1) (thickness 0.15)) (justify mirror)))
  (fp_rect (start 0 0) (end 39 -22.5) (stroke (width 0.3) (type solid)) (fill no) (layer "F.SilkS"))
  (pad "" thru_hole circle (at 7.9 -20.3 90) (size 2.54 2.54) (drill 2) (layers "*.Cu" "*.Mask") (remove_unused_layers no)
   (solder_mask_margin 0.127))
  (pad "" thru_hole circle (at 7.9 -2.3 90) (size 2.54 2.54) (drill 2) (layers "*.Cu" "*.Mask") (remove_unused_layers no)
   (solder_mask_margin 0.127))
  (pad "" thru_hole circle (at 34.4 -2.3 90) (size 2.54 2.54) (drill 2) (layers "*.Cu" "*.Mask") (remove_unused_layers no)
   (solder_mask_margin 0.127))
  (pad "7" thru_hole rect (at 37.5 -7.5 90) (size 2 2) (drill 1) (layers "*.Cu" "*.Mask") (remove_unused_layers no) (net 4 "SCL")
   (solder_mask_margin 0.127))
  (pad "8" thru_hole oval (at 37.5 -10.04 90) (size 2 2) (drill 1) (layers "*.Cu" "*.Mask") (remove_unused_layers no) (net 3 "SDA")
   (solder_mask_margin 0.127))
  (pad "9" thru_hole oval (at 37.5 -12.58 90) (size 2 2) (drill 1) (layers "*.Cu" "*.Mask") (remove_unused_layers no) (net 2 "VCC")
   (solder_mask_margin 0.127))
  (pad "10" thru_hole oval (at 37.5 -15.12 90) (size 2 2) (drill 1) (layers "*.Cu" "*.Mask") (remove_unused_layers no) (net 1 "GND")
   (solder_mask_margin 0.127)))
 (gr_rect (start 17.5 14) (end 83 73) (stroke (width 0.05) (type default)) (fill no) (layer "Edge.Cuts"))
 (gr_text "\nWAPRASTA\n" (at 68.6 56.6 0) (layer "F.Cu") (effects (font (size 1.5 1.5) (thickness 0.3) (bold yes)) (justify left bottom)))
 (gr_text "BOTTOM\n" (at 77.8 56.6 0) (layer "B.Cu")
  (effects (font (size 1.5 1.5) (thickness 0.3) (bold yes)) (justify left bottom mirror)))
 (segment (start 46.44 18.54) (end 46.44 18.48) (width 0.2) (layer "F.Cu") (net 6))
 (segment (start 47.75 22.95) (end 47.75 19.85) (width 0.3) (layer "F.Cu") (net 6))
 (segment (start 47.75 25.35) (end 47.7 25.4) (width 0.3) (layer "F.Cu") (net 6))
 (segment (start 47.75 22.95) (end 47.75 25.35) (width 1) (layer "F.Cu") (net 6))
 (segment (start 47.75 19.85) (end 46.44 18.54) (width 0.5) (layer "F.Cu") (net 6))
 (via (at 47.75 22.95) (size 1.524) (drill 1) (layers "F.Cu" "B.Cu") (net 6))
 (segment (start 46.44 18.48) (end 46.48 18.48) (width 0.2) (layer "B.Cu") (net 6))
 (segment (start 47.75 22.95) (end 47.75 27.54) (width 1) (layer "B.Cu") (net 6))
 (segment (start 47.75 27.54) (end 52.21 32) (width 1) (layer "B.Cu") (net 6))
 (segment (start 23.87 19.63) (end 25.02 18.48) (width 1) (layer "F.Cu") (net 2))
 (segment (start 23.87 22.77) (end 23.87 19.63) (width 1) (layer "F.Cu") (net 2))
 (segment (start 25.02 18.48) (end 26.12 18.48) (width 1) (layer "F.Cu") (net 2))
 (via (at 23.87 22.77) (size 1.524) (drill 1) (layers "F.Cu" "B.Cu") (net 2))
 (segment (start 33.7 43.6) (end 72.3 43.6) (width 1) (layer "B.Cu") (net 2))
 (segment (start 73.1 34.1) (end 76.2 37.2) (width 1) (layer "B.Cu") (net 2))
 (segment (start 56.21 32) (end 56.21 33.51) (width 1) (layer "B.Cu") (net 2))
 (segment (start 59.25 27.5) (end 56.21 30.54) (width 1) (layer "B.Cu") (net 2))
 (segment (start 71.75 27.5) (end 59.25 27.5) (width 1) (layer "B.Cu") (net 2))
 (segment (start 26.12 18.568925) (end 26.12 18.48) (width 0.4) (layer "B.Cu") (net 2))
 (segment (start 72.25 27.535) (end 71.785 27.535) (width 1) (layer "B.Cu") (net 2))
 (segment (start 56.8 34.1) (end 73.1 34.1) (width 1) (layer "B.Cu") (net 2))
 (segment (start 26.12 18.48) (end 26.03 18.39) (width 0.4) (layer "B.Cu") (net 2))
 (segment (start 23.87 22.77) (end 28.1 27) (width 1) (layer "B.Cu") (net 2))
 (segment (start 28.1 31.34) (end 28.16 31.4) (width 1) (layer "B.Cu") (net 2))
 (segment (start 28.1 27) (end 28.1 31.34) (width 1) (layer "B.Cu") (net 2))
 (segment (start 76.2 42.3) (end 74.9 43.6) (width 1) (layer "B.Cu") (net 2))
 (segment (start 56.21 30.54) (end 56.21 32) (width 1) (layer "B.Cu") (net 2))
 (segment (start 71.785 27.535) (end 71.75 27.5) (width 1) (layer "B.Cu") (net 2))
 (segment (start 28.16 38.06) (end 33.7 43.6) (width 1) (layer "B.Cu") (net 2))
 (segment (start 76.2 37.2) (end 76.2 42.3) (width 1) (layer "B.Cu") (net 2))
 (segment (start 56.21 33.51) (end 56.8 34.1) (width 1) (layer "B.Cu") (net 2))
 (segment (start 74.9 43.6) (end 72.3 43.6) (width 1) (layer "B.Cu") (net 2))
 (segment (start 28.16 31.4) (end 28.16 38.06) (width 1) (layer "B.Cu") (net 2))
 (segment (start 74.4 24.1) (end 74.4 21.04) (width 1) (layer "F.Cu") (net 1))
 (segment (start 74.4 21.04) (end 74.38 21.02) (width 1) (layer "F.Cu") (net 1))
 (via (at 74.4 24.1) (size 1.524) (drill 1) (layers "F.Cu" "B.Cu") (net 1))
 (segment (start 74.38 27.945) (end 74.38 24.12) (width 1) (layer "B.Cu") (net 1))
 (segment (start 25.56 31.34) (end 25.62 31.4) (width 0.2) (layer "B.Cu") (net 1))
 (segment (start 74.575 30.075) (end 79.9 35.4) (width 1) (layer "B.Cu") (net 1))
 (segment (start 72.3 46.1) (end 31.6 46.1) (width 1) (layer "B.Cu") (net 1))
 (segment (start 78.3 46.1) (end 72.3 46.1) (width 1) (layer "B.Cu") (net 1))
 (segment (start 72.25 30.075) (end 70.325 32) (width 1) (layer "B.Cu") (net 1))
 (segment (start 72.25 30.075) (end 74.38 27.945) (width 1) (layer "B.Cu") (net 1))
 (segment (start 72.25 30.075) (end 74.575 30.075) (width 1) (layer "B.Cu") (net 1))
 (segment (start 79.9 44.5) (end 78.3 46.1) (width 1) (layer "B.Cu") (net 1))
 (segment (start 58.21 32) (end 70.325 32) (width 1) (layer "B.Cu") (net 1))
 (segment (start 25.61 40.11) (end 25.61 31.4) (width 1) (layer "B.Cu") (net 1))
 (segment (start 31.6 46.1) (end 25.61 40.11) (width 1) (layer "B.Cu") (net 1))
 (segment (start 79.9 35.4) (end 79.9 44.5) (width 1) (layer "B.Cu") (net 1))
 (segment (start 74.38 24.12) (end 74.4 24.1) (width 1) (layer "B.Cu") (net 1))
 (segment (start 28.66 23.77) (end 28.66 21.02) (width 1) (layer "F.Cu") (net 3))
 (via (at 28.66 23.77) (size 1.524) (drill 1) (layers "F.Cu" "B.Cu") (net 3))
 (segment (start 72 41.4) (end 72.3 41.1) (width 1) (layer "B.Cu") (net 3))
 (segment (start 30.7 31.4) (end 30.7 36.5) (width 1) (layer "B.Cu") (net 3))
 (segment (start 30.64 31.34) (end 30.7 31.4) (width 0.2) (layer "B.Cu") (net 3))
 (segment (start 28.66 21.02) (end 29 21.36) (width 0.2) (layer "B.Cu") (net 3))
 (segment (start 30.64 25.75) (end 30.64 31.34) (width 1) (layer "B.Cu") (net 3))
 (segment (start 28.66 23.77) (end 30.64 25.75) (width 1) (layer "B.Cu") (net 3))
 (segment (start 30.7 36.5) (end 35.6 41.4) (width 1) (layer "B.Cu") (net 3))
 (segment (start 35.6 41.4) (end 72 41.4) (width 1) (layer "B.Cu") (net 3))
 (segment (start 33.2 24.4) (end 31.2 22.4) (width 1) (layer "F.Cu") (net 4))
 (segment (start 31.2 22.4) (end 31.2 21.02) (width 1) (layer "F.Cu") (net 4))
 (via (at 33.2 24.4) (size 1.524) (drill 1) (layers "F.Cu" "B.Cu") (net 4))
 (segment (start 33.18 31.34) (end 33.18 24.42) (width 1) (layer "B.Cu") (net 4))
 (segment (start 69.7 36) (end 72.3 38.6) (width 1) (layer "B.Cu") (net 4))
 (segment (start 51.1 36) (end 69.7 36) (width 1) (layer "B.Cu") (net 4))
 (segment (start 33.24 31.4) (end 46.5 31.4) (width 1) (layer "B.Cu") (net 4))
 (segment (start 46.5 31.4) (end 51.1 36) (width 1) (layer "B.Cu") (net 4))
 (segment (start 33.18 31.34) (end 33.24 31.34) (width 0.2) (layer "B.Cu") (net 4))
 (segment (start 33.18 24.42) (end 33.2 24.4) (width 1) (layer "B.Cu") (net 4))
 (segment (start 33.24 31.34) (end 33.24 31.4) (width 0.2) (layer "B.Cu") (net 4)))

